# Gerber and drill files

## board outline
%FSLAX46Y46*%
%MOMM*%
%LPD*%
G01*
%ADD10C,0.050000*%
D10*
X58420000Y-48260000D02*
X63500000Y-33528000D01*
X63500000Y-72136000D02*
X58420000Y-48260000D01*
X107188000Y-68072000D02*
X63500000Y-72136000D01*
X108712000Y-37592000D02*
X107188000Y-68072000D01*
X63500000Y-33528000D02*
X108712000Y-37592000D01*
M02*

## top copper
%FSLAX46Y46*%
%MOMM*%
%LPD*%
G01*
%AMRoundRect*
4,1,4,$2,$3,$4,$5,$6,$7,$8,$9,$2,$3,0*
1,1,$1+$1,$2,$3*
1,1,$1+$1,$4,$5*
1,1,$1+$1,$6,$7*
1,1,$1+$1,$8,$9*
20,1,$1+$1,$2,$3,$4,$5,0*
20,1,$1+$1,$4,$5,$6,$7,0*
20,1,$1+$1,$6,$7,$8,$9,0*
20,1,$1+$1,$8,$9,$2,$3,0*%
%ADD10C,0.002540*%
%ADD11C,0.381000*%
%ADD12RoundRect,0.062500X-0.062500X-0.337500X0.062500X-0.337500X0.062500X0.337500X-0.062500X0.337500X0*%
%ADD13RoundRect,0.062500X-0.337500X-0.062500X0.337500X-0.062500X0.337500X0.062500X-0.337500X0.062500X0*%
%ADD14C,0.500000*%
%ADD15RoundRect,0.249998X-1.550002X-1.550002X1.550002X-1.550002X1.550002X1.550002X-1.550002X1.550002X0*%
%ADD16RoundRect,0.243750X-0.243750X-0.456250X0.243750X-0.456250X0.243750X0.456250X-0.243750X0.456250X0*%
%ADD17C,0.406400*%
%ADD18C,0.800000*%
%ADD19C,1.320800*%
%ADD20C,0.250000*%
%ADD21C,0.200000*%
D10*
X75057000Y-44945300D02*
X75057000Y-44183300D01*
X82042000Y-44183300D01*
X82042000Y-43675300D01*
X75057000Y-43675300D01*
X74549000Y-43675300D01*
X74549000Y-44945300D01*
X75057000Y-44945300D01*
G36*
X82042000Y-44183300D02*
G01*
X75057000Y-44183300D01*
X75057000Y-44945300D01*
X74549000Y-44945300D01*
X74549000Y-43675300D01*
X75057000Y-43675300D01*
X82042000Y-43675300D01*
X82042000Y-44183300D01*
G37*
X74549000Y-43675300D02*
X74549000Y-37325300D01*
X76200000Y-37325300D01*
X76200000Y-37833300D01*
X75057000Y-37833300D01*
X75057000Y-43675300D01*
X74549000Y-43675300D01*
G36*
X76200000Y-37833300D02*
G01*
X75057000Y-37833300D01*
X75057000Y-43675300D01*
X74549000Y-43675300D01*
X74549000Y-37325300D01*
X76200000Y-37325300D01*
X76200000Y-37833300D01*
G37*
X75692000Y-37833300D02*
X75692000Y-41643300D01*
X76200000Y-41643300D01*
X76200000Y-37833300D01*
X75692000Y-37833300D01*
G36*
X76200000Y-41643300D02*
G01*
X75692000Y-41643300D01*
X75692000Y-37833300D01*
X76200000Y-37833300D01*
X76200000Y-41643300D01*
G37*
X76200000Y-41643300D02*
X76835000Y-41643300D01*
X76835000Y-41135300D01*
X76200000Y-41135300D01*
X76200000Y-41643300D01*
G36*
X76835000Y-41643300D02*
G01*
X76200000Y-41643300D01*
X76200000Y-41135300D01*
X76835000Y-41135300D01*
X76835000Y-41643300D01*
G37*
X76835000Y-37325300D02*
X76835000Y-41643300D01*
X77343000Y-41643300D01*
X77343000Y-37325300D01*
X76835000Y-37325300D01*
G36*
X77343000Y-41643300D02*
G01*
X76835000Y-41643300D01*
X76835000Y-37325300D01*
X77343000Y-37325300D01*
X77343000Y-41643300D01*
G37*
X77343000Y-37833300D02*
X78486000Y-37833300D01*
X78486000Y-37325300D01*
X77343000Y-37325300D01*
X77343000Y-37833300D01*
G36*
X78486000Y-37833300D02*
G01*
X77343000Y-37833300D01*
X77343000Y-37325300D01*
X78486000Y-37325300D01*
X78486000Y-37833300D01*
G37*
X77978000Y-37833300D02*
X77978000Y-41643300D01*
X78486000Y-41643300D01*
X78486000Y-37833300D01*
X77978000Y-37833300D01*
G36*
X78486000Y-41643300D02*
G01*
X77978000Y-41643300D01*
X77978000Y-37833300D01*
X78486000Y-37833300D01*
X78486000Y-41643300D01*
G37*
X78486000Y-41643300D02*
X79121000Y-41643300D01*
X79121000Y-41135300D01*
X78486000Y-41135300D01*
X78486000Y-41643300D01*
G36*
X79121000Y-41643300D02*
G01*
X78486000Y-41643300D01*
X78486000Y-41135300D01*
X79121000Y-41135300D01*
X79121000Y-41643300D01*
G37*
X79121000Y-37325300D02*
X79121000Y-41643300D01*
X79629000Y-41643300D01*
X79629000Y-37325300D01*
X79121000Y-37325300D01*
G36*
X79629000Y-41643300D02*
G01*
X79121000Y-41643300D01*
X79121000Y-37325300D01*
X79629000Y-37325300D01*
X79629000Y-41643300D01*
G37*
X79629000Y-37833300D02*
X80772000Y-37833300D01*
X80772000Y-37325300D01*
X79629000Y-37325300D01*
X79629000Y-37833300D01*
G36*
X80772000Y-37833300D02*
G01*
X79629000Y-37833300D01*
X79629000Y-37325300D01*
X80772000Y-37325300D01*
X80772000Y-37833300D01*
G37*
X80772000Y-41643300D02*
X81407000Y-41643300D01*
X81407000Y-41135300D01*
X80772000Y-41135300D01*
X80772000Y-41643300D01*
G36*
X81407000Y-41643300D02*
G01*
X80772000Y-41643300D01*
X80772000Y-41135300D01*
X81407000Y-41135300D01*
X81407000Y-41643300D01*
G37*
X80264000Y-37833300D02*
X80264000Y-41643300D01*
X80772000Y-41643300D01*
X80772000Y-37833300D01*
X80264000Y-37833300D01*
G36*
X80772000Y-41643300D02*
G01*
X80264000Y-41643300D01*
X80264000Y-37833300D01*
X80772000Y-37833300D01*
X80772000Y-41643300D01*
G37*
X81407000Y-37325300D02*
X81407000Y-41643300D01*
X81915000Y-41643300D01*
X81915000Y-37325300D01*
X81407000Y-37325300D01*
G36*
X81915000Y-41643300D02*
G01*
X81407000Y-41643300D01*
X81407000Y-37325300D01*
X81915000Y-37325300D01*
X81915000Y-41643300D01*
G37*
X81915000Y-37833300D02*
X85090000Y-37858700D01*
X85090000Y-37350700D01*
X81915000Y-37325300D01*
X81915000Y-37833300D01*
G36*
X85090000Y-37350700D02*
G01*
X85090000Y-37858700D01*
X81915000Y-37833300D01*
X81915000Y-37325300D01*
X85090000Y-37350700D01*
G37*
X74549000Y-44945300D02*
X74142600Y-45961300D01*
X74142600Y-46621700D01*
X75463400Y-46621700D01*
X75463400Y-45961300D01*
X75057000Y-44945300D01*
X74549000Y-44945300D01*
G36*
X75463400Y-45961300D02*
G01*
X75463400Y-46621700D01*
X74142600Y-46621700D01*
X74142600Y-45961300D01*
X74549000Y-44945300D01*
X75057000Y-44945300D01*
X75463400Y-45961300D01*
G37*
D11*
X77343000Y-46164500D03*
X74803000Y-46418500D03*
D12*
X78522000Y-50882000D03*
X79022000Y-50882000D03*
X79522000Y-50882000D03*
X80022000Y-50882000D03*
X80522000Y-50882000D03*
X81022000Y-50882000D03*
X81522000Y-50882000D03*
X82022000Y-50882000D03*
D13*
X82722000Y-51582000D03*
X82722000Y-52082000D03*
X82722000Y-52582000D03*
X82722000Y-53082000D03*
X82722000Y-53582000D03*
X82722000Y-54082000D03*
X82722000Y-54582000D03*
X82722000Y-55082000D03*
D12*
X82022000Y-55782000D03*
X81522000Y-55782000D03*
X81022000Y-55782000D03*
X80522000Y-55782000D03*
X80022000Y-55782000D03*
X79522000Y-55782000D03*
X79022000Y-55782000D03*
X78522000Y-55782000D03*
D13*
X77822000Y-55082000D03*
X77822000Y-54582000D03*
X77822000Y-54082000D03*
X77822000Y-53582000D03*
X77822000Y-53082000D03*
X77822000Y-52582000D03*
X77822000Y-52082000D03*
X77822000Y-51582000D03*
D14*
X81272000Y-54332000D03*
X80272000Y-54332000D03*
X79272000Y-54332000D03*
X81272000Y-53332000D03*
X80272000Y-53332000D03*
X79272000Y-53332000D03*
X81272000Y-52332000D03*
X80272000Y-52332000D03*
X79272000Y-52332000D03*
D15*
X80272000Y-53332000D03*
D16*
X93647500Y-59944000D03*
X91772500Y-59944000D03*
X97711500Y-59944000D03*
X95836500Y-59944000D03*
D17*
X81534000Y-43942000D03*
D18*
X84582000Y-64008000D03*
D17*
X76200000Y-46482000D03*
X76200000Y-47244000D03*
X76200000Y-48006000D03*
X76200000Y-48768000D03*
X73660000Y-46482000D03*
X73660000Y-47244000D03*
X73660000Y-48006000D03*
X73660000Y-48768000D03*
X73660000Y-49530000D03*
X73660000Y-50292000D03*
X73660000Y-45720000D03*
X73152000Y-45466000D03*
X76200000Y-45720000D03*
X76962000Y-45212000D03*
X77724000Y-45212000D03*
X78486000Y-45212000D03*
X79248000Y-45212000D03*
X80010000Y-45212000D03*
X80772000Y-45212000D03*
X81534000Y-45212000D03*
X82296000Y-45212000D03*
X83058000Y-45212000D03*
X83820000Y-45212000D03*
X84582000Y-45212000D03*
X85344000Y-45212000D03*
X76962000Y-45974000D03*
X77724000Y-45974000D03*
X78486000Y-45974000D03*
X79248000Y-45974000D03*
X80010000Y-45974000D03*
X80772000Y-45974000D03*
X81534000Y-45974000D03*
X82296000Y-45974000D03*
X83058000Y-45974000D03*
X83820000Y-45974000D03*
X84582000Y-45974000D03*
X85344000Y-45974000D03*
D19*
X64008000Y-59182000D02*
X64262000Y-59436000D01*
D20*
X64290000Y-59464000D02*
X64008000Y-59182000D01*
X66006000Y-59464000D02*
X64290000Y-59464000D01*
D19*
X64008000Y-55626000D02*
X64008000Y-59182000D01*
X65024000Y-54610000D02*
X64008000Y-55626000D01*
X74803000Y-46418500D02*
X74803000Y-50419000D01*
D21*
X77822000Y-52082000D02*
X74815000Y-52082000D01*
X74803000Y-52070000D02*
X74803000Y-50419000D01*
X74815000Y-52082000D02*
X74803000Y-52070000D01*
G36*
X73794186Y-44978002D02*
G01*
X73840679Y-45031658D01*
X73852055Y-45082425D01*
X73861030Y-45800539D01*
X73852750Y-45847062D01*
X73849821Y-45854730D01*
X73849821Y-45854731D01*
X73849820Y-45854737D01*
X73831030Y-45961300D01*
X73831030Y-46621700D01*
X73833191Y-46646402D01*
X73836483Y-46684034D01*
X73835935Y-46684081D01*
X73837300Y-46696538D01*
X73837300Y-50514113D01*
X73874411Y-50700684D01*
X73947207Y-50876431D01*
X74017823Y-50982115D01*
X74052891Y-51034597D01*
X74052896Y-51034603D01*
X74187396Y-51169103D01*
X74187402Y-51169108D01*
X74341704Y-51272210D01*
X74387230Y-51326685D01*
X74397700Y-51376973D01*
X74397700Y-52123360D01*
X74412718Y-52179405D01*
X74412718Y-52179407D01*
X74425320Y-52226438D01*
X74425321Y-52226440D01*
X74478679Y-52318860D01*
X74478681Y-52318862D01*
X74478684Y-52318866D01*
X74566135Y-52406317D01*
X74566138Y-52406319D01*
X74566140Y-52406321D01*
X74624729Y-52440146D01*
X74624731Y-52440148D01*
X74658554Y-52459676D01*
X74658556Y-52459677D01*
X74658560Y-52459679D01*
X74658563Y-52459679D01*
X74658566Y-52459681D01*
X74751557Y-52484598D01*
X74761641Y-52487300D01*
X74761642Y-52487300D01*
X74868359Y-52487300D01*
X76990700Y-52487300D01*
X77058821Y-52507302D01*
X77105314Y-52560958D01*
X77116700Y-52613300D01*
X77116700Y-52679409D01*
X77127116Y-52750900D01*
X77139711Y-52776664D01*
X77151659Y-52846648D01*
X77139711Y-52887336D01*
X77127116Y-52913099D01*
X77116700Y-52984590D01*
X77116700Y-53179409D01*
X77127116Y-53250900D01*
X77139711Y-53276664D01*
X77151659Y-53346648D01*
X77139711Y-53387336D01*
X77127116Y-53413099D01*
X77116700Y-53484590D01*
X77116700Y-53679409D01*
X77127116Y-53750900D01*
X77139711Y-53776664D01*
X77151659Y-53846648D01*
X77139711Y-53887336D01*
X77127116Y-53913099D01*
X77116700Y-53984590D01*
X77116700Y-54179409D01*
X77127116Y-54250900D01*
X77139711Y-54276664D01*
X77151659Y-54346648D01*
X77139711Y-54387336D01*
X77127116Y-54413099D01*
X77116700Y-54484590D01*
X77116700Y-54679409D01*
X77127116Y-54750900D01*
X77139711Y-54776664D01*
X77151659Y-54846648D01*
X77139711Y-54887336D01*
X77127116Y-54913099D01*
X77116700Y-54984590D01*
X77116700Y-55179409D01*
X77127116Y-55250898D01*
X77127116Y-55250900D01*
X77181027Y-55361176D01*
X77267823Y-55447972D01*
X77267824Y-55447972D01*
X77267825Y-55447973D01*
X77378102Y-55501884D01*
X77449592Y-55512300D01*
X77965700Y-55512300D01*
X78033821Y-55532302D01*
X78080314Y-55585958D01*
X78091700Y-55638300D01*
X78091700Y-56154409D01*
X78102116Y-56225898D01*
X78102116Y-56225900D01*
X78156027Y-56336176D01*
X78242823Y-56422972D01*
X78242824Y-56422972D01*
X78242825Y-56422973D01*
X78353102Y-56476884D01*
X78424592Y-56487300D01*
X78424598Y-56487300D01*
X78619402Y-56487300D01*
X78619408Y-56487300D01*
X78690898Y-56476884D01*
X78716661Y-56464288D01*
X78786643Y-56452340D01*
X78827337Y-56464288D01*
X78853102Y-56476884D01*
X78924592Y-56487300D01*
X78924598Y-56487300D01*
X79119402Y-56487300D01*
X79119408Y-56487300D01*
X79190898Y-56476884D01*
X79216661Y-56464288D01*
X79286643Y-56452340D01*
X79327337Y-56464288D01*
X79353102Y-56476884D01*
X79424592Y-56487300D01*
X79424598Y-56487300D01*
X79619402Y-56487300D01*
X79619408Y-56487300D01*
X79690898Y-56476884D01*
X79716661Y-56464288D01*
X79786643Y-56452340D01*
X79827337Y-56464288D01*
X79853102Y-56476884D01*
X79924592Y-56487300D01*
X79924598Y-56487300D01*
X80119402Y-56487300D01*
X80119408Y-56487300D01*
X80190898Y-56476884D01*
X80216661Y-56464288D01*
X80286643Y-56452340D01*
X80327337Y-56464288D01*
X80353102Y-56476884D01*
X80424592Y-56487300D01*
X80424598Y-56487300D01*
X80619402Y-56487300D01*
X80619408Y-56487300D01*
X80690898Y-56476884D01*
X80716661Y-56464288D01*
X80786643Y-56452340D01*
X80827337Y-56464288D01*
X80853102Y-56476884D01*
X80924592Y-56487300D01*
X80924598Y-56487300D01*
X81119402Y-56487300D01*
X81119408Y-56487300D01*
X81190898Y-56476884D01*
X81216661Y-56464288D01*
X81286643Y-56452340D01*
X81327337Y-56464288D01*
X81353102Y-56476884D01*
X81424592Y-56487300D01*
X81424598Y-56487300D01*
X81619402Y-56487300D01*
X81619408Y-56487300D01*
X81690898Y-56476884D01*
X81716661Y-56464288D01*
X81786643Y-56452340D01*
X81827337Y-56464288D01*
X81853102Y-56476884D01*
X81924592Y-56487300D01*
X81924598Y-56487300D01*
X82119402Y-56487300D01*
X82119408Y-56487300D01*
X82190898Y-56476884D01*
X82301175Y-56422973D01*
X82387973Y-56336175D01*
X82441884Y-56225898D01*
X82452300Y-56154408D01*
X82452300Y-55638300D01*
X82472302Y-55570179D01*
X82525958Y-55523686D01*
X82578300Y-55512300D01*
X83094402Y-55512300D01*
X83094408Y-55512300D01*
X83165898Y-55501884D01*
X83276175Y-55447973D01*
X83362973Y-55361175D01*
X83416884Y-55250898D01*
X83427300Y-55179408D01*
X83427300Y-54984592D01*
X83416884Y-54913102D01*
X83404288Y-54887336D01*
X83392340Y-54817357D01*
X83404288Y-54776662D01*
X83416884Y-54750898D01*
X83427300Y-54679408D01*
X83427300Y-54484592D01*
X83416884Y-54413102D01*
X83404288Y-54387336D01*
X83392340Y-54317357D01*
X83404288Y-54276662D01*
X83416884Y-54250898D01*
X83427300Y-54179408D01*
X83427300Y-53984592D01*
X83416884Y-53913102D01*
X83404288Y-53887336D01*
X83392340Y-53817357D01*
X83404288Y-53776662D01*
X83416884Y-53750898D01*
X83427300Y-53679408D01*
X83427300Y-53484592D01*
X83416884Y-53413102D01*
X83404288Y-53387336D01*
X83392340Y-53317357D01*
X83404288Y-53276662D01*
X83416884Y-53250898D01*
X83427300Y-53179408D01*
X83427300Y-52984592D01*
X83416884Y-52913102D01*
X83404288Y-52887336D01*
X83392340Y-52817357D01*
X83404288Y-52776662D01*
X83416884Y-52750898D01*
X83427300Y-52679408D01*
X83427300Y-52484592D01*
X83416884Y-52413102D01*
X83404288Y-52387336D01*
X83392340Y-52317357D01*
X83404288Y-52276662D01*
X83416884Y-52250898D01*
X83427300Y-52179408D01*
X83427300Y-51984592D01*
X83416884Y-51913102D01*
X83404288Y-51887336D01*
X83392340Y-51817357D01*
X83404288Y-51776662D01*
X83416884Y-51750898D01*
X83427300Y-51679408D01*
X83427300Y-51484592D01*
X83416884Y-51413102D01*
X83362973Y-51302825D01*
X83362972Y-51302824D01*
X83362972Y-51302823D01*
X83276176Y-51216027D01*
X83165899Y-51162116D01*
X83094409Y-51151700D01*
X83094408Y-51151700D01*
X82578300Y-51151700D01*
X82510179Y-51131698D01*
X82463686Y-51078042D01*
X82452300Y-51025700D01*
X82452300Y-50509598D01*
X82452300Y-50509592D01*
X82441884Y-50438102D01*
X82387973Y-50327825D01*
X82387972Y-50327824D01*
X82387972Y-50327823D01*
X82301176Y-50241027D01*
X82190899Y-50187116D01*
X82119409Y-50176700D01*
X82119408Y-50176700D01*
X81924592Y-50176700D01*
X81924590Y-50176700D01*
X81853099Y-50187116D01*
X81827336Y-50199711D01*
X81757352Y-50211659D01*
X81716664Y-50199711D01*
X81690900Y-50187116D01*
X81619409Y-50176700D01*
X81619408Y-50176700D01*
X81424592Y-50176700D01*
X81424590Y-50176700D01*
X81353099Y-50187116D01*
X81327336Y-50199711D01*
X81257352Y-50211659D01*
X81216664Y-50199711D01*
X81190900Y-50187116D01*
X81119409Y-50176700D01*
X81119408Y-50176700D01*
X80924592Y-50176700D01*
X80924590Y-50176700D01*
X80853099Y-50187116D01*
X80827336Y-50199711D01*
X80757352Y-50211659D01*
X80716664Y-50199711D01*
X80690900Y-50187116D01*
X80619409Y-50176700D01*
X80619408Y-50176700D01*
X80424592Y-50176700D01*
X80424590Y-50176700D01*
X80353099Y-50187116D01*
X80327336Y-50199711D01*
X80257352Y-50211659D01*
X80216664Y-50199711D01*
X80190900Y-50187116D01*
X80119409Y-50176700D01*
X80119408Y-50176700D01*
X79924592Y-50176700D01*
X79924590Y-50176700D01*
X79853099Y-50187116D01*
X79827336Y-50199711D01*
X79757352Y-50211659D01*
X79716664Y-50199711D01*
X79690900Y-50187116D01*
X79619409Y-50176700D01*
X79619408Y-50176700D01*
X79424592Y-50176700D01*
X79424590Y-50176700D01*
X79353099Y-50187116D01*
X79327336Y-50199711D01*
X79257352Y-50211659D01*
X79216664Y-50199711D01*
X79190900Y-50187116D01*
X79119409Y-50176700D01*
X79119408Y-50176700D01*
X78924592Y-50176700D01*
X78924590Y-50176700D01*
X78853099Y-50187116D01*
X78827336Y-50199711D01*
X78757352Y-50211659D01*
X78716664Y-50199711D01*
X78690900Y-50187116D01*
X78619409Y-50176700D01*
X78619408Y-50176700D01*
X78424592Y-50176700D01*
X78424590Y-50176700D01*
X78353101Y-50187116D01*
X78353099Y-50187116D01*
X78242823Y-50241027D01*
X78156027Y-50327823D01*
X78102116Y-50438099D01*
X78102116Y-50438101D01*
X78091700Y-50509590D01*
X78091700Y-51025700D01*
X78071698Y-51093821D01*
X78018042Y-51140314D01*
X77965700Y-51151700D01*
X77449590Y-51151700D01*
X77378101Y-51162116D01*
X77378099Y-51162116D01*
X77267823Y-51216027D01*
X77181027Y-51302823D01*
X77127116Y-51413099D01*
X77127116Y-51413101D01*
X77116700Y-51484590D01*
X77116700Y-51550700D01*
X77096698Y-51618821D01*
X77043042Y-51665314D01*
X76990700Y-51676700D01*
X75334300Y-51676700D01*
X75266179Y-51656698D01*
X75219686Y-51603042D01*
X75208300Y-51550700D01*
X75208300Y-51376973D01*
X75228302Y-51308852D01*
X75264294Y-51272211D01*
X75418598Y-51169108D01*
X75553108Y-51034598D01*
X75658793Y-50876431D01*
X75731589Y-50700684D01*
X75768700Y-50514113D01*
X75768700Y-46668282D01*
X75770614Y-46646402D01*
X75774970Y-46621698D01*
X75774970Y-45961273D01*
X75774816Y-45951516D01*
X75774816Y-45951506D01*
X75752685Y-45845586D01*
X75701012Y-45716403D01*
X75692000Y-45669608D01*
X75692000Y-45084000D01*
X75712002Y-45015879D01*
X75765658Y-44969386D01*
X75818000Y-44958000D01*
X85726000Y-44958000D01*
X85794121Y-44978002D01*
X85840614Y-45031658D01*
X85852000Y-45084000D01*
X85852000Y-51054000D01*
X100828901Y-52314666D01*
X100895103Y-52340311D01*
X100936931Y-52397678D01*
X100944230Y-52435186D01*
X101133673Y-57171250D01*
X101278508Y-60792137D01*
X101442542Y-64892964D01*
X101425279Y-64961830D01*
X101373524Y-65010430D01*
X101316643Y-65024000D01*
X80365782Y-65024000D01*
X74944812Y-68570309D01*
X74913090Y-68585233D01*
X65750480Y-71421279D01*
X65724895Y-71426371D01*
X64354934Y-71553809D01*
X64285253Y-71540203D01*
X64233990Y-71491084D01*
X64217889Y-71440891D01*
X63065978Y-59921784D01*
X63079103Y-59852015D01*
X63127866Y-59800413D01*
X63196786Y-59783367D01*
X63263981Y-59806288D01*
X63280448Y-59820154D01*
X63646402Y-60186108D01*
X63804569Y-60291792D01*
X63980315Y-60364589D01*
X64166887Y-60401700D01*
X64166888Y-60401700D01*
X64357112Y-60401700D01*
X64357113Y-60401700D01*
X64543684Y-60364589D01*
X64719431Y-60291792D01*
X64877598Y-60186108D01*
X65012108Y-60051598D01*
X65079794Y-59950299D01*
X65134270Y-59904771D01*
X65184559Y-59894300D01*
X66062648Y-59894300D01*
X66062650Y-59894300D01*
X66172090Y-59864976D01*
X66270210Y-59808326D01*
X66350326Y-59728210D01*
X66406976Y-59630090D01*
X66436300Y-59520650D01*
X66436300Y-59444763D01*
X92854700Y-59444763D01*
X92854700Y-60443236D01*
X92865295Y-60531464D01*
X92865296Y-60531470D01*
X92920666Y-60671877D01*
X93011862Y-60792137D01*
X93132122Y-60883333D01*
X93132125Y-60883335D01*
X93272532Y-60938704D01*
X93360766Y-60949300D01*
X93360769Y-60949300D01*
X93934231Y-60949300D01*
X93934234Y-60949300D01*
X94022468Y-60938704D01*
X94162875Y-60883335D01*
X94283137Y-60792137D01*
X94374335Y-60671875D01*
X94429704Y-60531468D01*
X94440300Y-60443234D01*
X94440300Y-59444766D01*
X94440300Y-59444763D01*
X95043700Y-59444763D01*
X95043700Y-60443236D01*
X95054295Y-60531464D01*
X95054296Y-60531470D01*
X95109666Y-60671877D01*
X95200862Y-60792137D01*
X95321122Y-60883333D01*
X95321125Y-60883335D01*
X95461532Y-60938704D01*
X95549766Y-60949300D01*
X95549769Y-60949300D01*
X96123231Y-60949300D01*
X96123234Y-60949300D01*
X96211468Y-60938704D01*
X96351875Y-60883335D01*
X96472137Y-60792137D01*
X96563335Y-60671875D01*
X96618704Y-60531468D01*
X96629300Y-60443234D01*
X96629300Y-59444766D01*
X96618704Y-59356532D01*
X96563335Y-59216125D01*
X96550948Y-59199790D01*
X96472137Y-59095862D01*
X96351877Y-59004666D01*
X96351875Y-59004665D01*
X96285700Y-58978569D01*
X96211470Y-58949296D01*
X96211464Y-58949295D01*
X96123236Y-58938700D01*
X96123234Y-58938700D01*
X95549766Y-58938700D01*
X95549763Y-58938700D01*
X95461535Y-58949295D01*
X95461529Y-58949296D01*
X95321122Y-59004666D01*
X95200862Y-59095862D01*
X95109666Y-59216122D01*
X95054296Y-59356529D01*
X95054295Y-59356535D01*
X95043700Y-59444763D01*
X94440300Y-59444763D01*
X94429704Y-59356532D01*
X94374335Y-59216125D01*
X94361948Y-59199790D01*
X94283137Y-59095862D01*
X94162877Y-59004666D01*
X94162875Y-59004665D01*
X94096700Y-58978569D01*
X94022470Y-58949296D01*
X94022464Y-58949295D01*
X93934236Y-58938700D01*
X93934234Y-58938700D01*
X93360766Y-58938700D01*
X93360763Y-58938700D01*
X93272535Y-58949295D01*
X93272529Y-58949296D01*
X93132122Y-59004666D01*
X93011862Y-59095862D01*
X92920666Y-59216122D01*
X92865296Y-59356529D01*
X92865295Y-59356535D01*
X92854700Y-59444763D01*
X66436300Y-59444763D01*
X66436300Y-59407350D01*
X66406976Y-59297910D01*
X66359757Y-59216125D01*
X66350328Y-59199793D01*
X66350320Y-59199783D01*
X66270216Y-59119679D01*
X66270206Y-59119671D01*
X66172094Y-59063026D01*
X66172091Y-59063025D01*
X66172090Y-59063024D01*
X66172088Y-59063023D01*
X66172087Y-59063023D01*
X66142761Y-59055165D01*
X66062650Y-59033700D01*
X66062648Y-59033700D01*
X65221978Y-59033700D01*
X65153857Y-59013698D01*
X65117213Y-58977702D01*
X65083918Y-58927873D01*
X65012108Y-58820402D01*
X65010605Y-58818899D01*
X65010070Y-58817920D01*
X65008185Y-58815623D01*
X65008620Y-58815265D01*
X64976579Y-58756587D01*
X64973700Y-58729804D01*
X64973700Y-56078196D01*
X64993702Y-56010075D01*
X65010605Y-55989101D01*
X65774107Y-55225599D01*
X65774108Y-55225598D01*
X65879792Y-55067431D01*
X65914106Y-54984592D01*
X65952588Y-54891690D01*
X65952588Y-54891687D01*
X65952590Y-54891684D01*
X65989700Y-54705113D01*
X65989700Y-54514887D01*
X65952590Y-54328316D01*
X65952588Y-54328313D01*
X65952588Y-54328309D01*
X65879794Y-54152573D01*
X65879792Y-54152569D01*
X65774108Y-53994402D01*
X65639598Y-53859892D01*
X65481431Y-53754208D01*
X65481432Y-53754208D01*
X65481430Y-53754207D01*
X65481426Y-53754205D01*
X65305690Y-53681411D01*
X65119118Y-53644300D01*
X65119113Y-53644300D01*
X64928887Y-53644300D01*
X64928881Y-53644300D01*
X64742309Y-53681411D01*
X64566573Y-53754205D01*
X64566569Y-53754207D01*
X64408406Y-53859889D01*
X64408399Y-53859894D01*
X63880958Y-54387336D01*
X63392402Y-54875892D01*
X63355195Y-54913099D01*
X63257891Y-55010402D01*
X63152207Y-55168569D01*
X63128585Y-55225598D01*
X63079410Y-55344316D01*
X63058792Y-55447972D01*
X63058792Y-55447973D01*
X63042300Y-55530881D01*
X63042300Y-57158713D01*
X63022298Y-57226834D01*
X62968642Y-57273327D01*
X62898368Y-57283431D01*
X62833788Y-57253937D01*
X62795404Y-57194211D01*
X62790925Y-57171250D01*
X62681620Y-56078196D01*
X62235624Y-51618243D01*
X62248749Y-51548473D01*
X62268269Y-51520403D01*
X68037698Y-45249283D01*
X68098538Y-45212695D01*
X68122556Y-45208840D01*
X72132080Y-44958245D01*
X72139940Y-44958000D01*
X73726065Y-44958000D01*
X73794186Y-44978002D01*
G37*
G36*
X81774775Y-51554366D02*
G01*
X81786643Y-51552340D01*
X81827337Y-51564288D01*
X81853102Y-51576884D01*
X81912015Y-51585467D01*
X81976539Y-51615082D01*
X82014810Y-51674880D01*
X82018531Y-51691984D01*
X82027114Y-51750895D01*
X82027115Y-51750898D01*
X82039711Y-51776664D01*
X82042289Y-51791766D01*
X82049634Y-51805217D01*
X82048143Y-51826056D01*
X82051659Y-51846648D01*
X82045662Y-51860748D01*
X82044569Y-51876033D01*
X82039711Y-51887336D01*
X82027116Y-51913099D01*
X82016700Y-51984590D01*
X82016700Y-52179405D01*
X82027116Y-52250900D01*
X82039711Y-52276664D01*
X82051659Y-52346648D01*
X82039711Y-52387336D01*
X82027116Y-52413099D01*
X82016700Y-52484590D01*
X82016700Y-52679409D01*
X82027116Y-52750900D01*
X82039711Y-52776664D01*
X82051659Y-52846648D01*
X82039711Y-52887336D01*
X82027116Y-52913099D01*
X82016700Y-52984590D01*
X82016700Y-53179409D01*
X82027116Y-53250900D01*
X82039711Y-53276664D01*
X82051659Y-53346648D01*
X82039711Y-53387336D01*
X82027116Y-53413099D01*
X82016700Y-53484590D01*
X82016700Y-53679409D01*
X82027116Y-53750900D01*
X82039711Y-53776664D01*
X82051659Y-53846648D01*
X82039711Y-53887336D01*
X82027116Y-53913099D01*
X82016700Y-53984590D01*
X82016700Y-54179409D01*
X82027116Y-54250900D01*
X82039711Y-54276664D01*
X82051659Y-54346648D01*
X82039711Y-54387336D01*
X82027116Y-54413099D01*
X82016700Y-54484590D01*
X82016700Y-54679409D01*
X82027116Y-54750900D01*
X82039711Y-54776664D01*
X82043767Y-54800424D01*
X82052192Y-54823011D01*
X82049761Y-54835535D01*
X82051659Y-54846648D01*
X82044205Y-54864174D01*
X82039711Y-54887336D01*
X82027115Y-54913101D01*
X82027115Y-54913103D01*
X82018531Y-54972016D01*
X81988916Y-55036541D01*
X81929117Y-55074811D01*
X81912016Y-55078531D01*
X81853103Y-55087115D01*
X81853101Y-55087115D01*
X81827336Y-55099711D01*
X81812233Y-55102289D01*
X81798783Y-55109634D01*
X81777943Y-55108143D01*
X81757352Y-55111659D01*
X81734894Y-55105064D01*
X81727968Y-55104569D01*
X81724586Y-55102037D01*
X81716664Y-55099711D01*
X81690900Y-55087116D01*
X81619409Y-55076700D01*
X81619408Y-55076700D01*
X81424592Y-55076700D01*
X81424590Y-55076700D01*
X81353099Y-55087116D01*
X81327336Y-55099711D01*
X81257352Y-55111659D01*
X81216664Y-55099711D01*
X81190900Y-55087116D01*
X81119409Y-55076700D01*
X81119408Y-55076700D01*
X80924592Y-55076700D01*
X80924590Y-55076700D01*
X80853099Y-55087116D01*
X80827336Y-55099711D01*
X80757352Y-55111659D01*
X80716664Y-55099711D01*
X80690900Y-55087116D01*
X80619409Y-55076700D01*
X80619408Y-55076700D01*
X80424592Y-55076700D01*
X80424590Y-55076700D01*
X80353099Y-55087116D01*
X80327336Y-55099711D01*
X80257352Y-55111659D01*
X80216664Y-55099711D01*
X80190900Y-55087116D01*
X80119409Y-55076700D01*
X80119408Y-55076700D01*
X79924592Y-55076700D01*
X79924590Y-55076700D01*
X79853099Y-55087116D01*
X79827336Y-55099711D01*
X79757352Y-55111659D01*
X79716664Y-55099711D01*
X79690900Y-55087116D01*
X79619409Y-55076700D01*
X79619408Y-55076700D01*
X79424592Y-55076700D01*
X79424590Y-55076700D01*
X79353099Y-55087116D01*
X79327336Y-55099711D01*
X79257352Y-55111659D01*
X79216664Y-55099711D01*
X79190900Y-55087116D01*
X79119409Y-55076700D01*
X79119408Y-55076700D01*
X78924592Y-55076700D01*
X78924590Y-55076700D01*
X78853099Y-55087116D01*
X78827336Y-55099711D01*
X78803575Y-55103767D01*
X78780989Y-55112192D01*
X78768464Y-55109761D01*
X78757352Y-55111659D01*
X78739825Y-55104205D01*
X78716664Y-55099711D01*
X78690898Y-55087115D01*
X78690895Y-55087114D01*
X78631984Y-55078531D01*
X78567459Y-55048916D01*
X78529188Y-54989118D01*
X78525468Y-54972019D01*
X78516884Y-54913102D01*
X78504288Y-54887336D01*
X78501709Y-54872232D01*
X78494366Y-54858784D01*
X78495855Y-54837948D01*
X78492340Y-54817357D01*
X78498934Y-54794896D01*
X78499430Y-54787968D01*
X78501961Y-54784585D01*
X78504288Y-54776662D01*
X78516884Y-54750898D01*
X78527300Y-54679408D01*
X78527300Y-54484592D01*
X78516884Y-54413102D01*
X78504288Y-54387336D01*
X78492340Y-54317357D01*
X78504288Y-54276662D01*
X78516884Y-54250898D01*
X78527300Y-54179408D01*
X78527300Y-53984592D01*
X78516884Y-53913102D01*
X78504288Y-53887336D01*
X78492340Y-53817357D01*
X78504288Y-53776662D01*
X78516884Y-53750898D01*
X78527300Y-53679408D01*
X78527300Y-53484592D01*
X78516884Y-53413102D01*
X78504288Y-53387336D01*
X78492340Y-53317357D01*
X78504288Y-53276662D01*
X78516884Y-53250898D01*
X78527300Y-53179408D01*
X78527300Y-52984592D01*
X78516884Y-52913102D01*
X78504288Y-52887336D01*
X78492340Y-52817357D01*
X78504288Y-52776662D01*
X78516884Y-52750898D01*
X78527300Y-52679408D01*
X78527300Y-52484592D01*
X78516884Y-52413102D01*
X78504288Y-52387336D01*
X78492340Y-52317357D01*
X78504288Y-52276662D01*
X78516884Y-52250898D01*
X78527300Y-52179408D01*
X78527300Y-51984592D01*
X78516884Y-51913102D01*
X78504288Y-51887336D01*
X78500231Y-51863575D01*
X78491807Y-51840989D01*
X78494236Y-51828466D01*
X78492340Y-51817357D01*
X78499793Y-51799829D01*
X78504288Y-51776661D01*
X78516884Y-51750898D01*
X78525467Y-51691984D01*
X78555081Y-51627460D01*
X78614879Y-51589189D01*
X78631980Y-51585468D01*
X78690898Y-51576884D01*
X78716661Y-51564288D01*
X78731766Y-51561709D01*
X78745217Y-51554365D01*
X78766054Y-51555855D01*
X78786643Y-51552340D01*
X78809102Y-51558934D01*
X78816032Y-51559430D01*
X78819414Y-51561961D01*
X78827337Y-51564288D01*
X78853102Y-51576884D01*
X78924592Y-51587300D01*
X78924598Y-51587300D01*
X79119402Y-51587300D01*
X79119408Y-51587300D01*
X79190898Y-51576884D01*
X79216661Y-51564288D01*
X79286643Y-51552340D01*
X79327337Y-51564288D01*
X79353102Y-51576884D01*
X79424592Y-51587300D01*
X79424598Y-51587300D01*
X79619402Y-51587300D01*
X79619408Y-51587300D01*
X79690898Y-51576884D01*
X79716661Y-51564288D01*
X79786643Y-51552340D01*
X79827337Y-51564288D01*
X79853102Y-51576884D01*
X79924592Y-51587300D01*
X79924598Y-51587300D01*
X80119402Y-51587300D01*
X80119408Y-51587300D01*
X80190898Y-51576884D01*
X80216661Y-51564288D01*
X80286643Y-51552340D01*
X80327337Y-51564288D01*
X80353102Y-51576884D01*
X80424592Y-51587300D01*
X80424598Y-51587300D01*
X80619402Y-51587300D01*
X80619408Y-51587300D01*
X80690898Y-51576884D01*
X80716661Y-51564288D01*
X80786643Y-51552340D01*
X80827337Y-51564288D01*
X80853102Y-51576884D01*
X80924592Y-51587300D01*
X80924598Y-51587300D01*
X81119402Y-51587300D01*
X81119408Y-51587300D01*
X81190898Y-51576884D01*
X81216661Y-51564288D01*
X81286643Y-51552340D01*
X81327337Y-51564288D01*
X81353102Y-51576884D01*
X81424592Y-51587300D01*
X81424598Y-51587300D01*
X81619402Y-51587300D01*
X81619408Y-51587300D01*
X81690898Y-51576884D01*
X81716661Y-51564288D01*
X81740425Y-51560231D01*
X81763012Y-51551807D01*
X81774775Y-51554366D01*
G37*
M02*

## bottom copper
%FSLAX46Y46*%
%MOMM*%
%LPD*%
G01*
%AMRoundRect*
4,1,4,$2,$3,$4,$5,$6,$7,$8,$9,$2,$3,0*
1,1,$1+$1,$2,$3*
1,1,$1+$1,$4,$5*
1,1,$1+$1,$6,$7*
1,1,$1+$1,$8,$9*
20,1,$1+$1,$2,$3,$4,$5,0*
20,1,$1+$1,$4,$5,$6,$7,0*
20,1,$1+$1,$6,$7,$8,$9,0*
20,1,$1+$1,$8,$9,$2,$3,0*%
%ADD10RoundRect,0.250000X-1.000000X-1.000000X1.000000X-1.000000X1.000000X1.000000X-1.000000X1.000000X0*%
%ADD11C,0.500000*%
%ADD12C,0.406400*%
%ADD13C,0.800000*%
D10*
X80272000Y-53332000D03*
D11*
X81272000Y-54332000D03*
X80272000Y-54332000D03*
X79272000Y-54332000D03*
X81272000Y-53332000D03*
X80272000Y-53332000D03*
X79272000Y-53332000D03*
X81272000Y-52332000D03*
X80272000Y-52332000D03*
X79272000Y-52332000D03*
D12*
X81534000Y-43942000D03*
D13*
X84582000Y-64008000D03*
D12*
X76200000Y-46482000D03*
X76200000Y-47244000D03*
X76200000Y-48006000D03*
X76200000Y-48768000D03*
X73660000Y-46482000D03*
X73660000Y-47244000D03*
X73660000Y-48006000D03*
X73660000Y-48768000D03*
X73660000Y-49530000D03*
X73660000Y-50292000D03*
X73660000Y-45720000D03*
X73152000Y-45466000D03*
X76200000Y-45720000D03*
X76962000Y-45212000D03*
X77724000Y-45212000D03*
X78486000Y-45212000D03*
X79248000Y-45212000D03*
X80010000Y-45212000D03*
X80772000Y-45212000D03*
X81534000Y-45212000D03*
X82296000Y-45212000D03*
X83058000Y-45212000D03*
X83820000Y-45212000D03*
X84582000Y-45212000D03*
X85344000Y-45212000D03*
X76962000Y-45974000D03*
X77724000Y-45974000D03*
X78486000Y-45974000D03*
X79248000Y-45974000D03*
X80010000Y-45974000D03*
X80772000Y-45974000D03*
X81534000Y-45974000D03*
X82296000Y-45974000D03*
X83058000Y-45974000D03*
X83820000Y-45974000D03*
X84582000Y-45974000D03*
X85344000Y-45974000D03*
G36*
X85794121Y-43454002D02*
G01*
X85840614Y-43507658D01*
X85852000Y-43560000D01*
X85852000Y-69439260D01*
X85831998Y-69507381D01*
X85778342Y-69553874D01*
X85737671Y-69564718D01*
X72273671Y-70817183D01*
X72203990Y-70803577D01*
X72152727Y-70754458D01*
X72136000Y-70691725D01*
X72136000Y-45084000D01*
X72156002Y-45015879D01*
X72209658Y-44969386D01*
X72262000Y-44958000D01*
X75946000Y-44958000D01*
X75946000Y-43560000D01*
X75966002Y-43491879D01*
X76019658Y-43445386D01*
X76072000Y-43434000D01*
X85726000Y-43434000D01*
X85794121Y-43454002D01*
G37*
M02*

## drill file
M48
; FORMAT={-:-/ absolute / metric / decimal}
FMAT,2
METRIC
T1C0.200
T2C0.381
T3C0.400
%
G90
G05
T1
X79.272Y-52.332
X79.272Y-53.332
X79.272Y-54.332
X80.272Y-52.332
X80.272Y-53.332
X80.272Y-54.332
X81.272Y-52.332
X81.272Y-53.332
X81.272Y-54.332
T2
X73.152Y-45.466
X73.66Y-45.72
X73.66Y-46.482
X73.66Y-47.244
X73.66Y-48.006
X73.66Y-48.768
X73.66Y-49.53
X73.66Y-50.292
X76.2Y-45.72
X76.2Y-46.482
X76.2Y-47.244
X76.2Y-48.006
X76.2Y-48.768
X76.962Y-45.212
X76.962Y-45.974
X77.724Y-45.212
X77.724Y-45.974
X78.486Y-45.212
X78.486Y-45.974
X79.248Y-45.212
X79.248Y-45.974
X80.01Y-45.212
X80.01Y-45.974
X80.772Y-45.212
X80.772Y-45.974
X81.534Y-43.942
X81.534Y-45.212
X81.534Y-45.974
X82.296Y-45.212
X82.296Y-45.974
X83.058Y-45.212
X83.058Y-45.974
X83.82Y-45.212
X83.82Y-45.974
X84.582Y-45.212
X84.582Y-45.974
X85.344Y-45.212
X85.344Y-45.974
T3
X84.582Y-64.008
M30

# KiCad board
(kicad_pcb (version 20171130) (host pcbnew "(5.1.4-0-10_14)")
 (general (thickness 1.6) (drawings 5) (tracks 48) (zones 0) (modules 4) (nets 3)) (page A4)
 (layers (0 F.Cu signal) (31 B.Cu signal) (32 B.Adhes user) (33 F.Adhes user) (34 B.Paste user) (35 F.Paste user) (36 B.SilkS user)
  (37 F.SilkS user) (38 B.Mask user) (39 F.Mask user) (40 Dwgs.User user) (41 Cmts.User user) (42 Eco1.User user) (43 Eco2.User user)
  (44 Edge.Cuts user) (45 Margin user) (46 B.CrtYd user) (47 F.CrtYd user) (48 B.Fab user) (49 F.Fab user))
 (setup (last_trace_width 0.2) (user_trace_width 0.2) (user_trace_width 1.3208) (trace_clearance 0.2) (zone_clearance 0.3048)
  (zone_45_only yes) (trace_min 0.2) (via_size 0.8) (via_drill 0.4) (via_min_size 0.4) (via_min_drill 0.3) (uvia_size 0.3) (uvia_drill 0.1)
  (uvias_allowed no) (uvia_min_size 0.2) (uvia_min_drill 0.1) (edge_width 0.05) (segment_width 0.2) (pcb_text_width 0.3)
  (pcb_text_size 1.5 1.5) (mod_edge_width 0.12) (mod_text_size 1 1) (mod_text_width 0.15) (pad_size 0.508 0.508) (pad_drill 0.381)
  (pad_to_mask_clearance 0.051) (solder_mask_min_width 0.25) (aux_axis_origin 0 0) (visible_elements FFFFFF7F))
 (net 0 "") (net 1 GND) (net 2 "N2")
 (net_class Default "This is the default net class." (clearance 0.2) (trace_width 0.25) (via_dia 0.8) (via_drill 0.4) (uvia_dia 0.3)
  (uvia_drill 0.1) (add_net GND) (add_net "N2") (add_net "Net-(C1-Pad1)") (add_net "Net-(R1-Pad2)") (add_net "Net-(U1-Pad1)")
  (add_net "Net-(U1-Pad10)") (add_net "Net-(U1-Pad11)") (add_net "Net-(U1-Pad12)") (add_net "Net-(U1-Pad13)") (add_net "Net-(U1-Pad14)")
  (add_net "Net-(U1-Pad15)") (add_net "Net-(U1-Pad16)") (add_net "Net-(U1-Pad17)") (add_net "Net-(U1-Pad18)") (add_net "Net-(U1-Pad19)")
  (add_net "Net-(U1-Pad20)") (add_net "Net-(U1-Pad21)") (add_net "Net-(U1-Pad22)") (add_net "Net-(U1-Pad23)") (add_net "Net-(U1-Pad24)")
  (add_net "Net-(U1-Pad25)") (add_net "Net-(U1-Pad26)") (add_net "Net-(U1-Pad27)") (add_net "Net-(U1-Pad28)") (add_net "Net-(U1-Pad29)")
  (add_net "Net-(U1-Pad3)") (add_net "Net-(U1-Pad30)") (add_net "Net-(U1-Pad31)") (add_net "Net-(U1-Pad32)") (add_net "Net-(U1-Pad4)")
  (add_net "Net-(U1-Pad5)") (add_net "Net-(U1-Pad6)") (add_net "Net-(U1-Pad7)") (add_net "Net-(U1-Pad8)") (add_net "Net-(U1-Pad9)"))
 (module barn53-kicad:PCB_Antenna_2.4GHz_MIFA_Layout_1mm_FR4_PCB (layer F.Cu) (at 74.803 46.4185)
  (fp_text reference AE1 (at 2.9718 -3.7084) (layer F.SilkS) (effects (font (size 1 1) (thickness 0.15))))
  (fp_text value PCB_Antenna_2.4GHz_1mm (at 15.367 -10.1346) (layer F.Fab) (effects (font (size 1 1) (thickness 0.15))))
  (fp_poly
   (pts (xy 0.254 -1.4732) (xy 0.254 -2.2352) (xy 7.239 -2.2352) (xy 7.239 -2.7432) (xy 0.254 -2.7432) (xy -0.254 -2.7432)
    (xy -0.254 -1.4732))
   (layer F.Cu) (width 0.00254))
  (fp_poly
   (pts (xy -0.254 -2.7432) (xy -0.254 -9.0932) (xy 1.397 -9.0932) (xy 1.397 -8.5852) (xy 0.254 -8.5852) (xy 0.254 -2.7432)) (layer F.Cu)
   (width 0.00254))
  (fp_poly (pts (xy 0.889 -8.5852) (xy 0.889 -4.7752) (xy 1.397 -4.7752) (xy 1.397 -8.5852)) (layer F.Cu) (width 0.00254))
  (fp_poly (pts (xy 1.397 -4.7752) (xy 2.032 -4.7752) (xy 2.032 -5.2832) (xy 1.397 -5.2832)) (layer F.Cu) (width 0.00254))
  (fp_poly (pts (xy 2.032 -9.0932) (xy 2.032 -4.7752) (xy 2.54 -4.7752) (xy 2.54 -9.0932)) (layer F.Cu) (width 0.00254))
  (fp_poly (pts (xy 2.54 -8.5852) (xy 3.683 -8.5852) (xy 3.683 -9.0932) (xy 2.54 -9.0932)) (layer F.Cu) (width 0.00254))
  (fp_poly (pts (xy 3.175 -8.5852) (xy 3.175 -4.7752) (xy 3.683 -4.7752) (xy 3.683 -8.5852)) (layer F.Cu) (width 0.00254))
  (fp_poly (pts (xy 3.683 -4.7752) (xy 4.318 -4.7752) (xy 4.318 -5.2832) (xy 3.683 -5.2832)) (layer F.Cu) (width 0.00254))
  (fp_poly (pts (xy 4.318 -9.0932) (xy 4.318 -4.7752) (xy 4.826 -4.7752) (xy 4.826 -9.0932)) (layer F.Cu) (width 0.00254))
  (fp_poly (pts (xy 4.826 -8.5852) (xy 5.969 -8.5852) (xy 5.969 -9.0932) (xy 4.826 -9.0932)) (layer F.Cu) (width 0.00254))
  (fp_poly (pts (xy 5.969 -4.7752) (xy 6.604 -4.7752) (xy 6.604 -5.2832) (xy 5.969 -5.2832)) (layer F.Cu) (width 0.00254))
  (fp_poly (pts (xy 5.461 -8.5852) (xy 5.461 -4.7752) (xy 5.969 -4.7752) (xy 5.969 -8.5852)) (layer F.Cu) (width 0.00254))
  (fp_poly (pts (xy 6.604 -9.0932) (xy 6.604 -4.7752) (xy 7.112 -4.7752) (xy 7.112 -9.0932)) (layer F.Cu) (width 0.00254))
  (fp_poly (pts (xy 7.112 -8.5852) (xy 10.287 -8.5598) (xy 10.287 -9.0678) (xy 7.112 -9.0932)) (layer F.Cu) (width 0.00254))
  (fp_poly
   (pts (xy -0.254 -1.4732) (xy -0.6604 -0.4572) (xy -0.6604 0.2032) (xy 0.6604 0.2032) (xy 0.6604 -0.4572) (xy 0.254 -1.4732)) (layer F.Cu)
   (width 0.00254))
  (pad 2 connect circle (at 2.54 -0.254) (size 0.381 0.381) (layers F.Cu) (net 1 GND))
  (pad 1 connect circle (at 0 0) (size 0.381 0.381) (layers F.Cu) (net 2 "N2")))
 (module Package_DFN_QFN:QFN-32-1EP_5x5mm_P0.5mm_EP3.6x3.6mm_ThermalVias (layer F.Cu) (at 80.272 53.332)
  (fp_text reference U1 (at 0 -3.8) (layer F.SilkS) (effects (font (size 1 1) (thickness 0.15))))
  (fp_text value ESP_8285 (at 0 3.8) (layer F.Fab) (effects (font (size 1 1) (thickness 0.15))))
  (pad 32 smd roundrect (at -1.75 -2.45) (size 0.25 0.8) (layers F.Cu F.Paste F.Mask) (roundrect_rratio 0.25))
  (pad 31 smd roundrect (at -1.25 -2.45) (size 0.25 0.8) (layers F.Cu F.Paste F.Mask) (roundrect_rratio 0.25))
  (pad 30 smd roundrect (at -0.75 -2.45) (size 0.25 0.8) (layers F.Cu F.Paste F.Mask) (roundrect_rratio 0.25))
  (pad 29 smd roundrect (at -0.25 -2.45) (size 0.25 0.8) (layers F.Cu F.Paste F.Mask) (roundrect_rratio 0.25))
  (pad 28 smd roundrect (at 0.25 -2.45) (size 0.25 0.8) (layers F.Cu F.Paste F.Mask) (roundrect_rratio 0.25))
  (pad 27 smd roundrect (at 0.75 -2.45) (size 0.25 0.8) (layers F.Cu F.Paste F.Mask) (roundrect_rratio 0.25))
  (pad 26 smd roundrect (at 1.25 -2.45) (size 0.25 0.8) (layers F.Cu F.Paste F.Mask) (roundrect_rratio 0.25))
  (pad 25 smd roundrect (at 1.75 -2.45) (size 0.25 0.8) (layers F.Cu F.Paste F.Mask) (roundrect_rratio 0.25))
  (pad 24 smd roundrect (at 2.45 -1.75) (size 0.8 0.25) (layers F.Cu F.Paste F.Mask) (roundrect_rratio 0.25))
  (pad 23 smd roundrect (at 2.45 -1.25) (size 0.8 0.25) (layers F.Cu F.Paste F.Mask) (roundrect_rratio 0.25))
  (pad 22 smd roundrect (at 2.45 -0.75) (size 0.8 0.25) (layers F.Cu F.Paste F.Mask) (roundrect_rratio 0.25))
  (pad 21 smd roundrect (at 2.45 -0.25) (size 0.8 0.25) (layers F.Cu F.Paste F.Mask) (roundrect_rratio 0.25))
  (pad 20 smd roundrect (at 2.45 0.25) (size 0.8 0.25) (layers F.Cu F.Paste F.Mask) (roundrect_rratio 0.25))
  (pad 19 smd roundrect (at 2.45 0.75) (size 0.8 0.25) (layers F.Cu F.Paste F.Mask) (roundrect_rratio 0.25))
  (pad 18 smd roundrect (at 2.45 1.25) (size 0.8 0.25) (layers F.Cu F.Paste F.Mask) (roundrect_rratio 0.25))
  (pad 17 smd roundrect (at 2.45 1.75) (size 0.8 0.25) (layers F.Cu F.Paste F.Mask) (roundrect_rratio 0.25))
  (pad 16 smd roundrect (at 1.75 2.45) (size 0.25 0.8) (layers F.Cu F.Paste F.Mask) (roundrect_rratio 0.25))
  (pad 15 smd roundrect (at 1.25 2.45) (size 0.25 0.8) (layers F.Cu F.Paste F.Mask) (roundrect_rratio 0.25))
  (pad 14 smd roundrect (at 0.75 2.45) (size 0.25 0.8) (layers F.Cu F.Paste F.Mask) (roundrect_rratio 0.25))
  (pad 13 smd roundrect (at 0.25 2.45) (size 0.25 0.8) (layers F.Cu F.Paste F.Mask) (roundrect_rratio 0.25))
  (pad 12 smd roundrect (at -0.25 2.45) (size 0.25 0.8) (layers F.Cu F.Paste F.Mask) (roundrect_rratio 0.25))
  (pad 11 smd roundrect (at -0.75 2.45) (size 0.25 0.8) (layers F.Cu F.Paste F.Mask) (roundrect_rratio 0.25))
  (pad 10 smd roundrect (at -1.25 2.45) (size 0.25 0.8) (layers F.Cu F.Paste F.Mask) (roundrect_rratio 0.25))
  (pad 9 smd roundrect (at -1.75 2.45) (size 0.25 0.8) (layers F.Cu F.Paste F.Mask) (roundrect_rratio 0.25))
  (pad 8 smd roundrect (at -2.45 1.75) (size 0.8 0.25) (layers F.Cu F.Paste F.Mask) (roundrect_rratio 0.25))
  (pad 7 smd roundrect (at -2.45 1.25) (size 0.8 0.25) (layers F.Cu F.Paste F.Mask) (roundrect_rratio 0.25))
  (pad 6 smd roundrect (at -2.45 0.75) (size 0.8 0.25) (layers F.Cu F.Paste F.Mask) (roundrect_rratio 0.25))
  (pad 5 smd roundrect (at -2.45 0.25) (size 0.8 0.25) (layers F.Cu F.Paste F.Mask) (roundrect_rratio 0.25))
  (pad 4 smd roundrect (at -2.45 -0.25) (size 0.8 0.25) (layers F.Cu F.Paste F.Mask) (roundrect_rratio 0.25))
  (pad 3 smd roundrect (at -2.45 -0.75) (size 0.8 0.25) (layers F.Cu F.Paste F.Mask) (roundrect_rratio 0.25))
  (pad 2 smd roundrect (at -2.45 -1.25) (size 0.8 0.25) (layers F.Cu F.Paste F.Mask) (roundrect_rratio 0.25) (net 2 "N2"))
  (pad 1 smd roundrect (at -2.45 -1.75) (size 0.8 0.25) (layers F.Cu F.Paste F.Mask) (roundrect_rratio 0.25))
  (pad "" smd custom (at 1.4 1.4) (size 0.554596 0.554596) (layers F.Paste) (options (clearance outline) (anchor circle)) (primitives))
  (pad "" smd custom (at 1.4 -1.4) (size 0.554596 0.554596) (layers F.Paste) (options (clearance outline) (anchor circle)) (primitives))
  (pad "" smd custom (at -1.4 1.4) (size 0.554596 0.554596) (layers F.Paste) (options (clearance outline) (anchor circle)) (primitives))
  (pad "" smd custom (at -1.4 -1.4) (size 0.554596 0.554596) (layers F.Paste) (options (clearance outline) (anchor circle)) (primitives))
  (pad "" smd custom (at 0.5 1.4) (size 0.568298 0.568298) (layers F.Paste) (options (clearance outline) (anchor circle)) (primitives))
  (pad "" smd custom (at -0.5 1.4) (size 0.568298 0.568298) (layers F.Paste) (options (clearance outline) (anchor circle)) (primitives))
  (pad "" smd custom (at 0.5 -1.4) (size 0.568298 0.568298) (layers F.Paste) (options (clearance outline) (anchor circle)) (primitives))
  (pad "" smd custom (at -0.5 -1.4) (size 0.568298 0.568298) (layers F.Paste) (options (clearance outline) (anchor circle)) (primitives))
  (pad "" smd custom (at 1.4 0.5) (size 0.568298 0.568298) (layers F.Paste) (options (clearance outline) (anchor circle)) (primitives))
  (pad "" smd custom (at 1.4 -0.5) (size 0.568298 0.568298) (layers F.Paste) (options (clearance outline) (anchor circle)) (primitives))
  (pad "" smd custom (at -1.4 0.5) (size 0.568298 0.568298) (layers F.Paste) (options (clearance outline) (anchor circle)) (primitives))
  (pad "" smd custom (at -1.4 -0.5) (size 0.568298 0.568298) (layers F.Paste) (options (clearance outline) (anchor circle)) (primitives))
  (pad "" smd roundrect (at 0.5 0.5) (size 0.806226 0.806226) (layers F.Paste) (roundrect_rratio 0.25))
  (pad "" smd roundrect (at 0.5 -0.5) (size 0.806226 0.806226) (layers F.Paste) (roundrect_rratio 0.25))
  (pad "" smd roundrect (at -0.5 0.5) (size 0.806226 0.806226) (layers F.Paste) (roundrect_rratio 0.25))
  (pad "" smd roundrect (at -0.5 -0.5) (size 0.806226 0.806226) (layers F.Paste) (roundrect_rratio 0.25))
  (pad 33 smd roundrect (at 0 0) (size 2.5 2.5) (layers B.Cu) (roundrect_rratio 0.1) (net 1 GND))
  (pad 33 thru_hole circle (at 1 1) (size 0.5 0.5) (drill 0.2) (layers *.Cu) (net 1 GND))
  (pad 33 thru_hole circle (at 0 1) (size 0.5 0.5) (drill 0.2) (layers *.Cu) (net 1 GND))
  (pad 33 thru_hole circle (at -1 1) (size 0.5 0.5) (drill 0.2) (layers *.Cu) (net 1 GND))
  (pad 33 thru_hole circle (at 1 0) (size 0.5 0.5) (drill 0.2) (layers *.Cu) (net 1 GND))
  (pad 33 thru_hole circle (at 0 0) (size 0.5 0.5) (drill 0.2) (layers *.Cu) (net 1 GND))
  (pad 33 thru_hole circle (at -1 0) (size 0.5 0.5) (drill 0.2) (layers *.Cu) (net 1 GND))
  (pad 33 thru_hole circle (at 1 -1) (size 0.5 0.5) (drill 0.2) (layers *.Cu) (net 1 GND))
  (pad 33 thru_hole circle (at 0 -1) (size 0.5 0.5) (drill 0.2) (layers *.Cu) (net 1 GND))
  (pad 33 thru_hole circle (at -1 -1) (size 0.5 0.5) (drill 0.2) (layers *.Cu) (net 1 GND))
  (pad 33 smd roundrect (at 0 0) (size 3.6 3.6) (layers F.Cu F.Mask) (roundrect_rratio 0.06944400000000001) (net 1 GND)))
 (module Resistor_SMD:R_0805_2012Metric (layer F.Cu) (at 92.71 59.944)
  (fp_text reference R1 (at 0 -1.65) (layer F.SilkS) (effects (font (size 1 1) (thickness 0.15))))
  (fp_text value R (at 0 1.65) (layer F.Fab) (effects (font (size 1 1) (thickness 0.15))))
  (pad 2 smd roundrect (at 0.9375 0) (size 0.975 1.4) (layers F.Cu F.Paste F.Mask) (roundrect_rratio 0.25))
  (pad 1 smd roundrect (at -0.9375 0) (size 0.975 1.4) (layers F.Cu F.Paste F.Mask) (roundrect_rratio 0.25) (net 1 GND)))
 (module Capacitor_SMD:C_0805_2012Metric (layer F.Cu) (at 96.774 59.944)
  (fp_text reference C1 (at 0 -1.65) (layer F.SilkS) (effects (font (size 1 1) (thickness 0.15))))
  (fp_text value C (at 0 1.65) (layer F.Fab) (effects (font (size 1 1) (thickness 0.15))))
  (pad 2 smd roundrect (at 0.9375 0) (size 0.975 1.4) (layers F.Cu F.Paste F.Mask) (roundrect_rratio 0.25) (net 1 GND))
  (pad 1 smd roundrect (at -0.9375 0) (size 0.975 1.4) (layers F.Cu F.Paste F.Mask) (roundrect_rratio 0.25)))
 (gr_line (start 58.42 48.26) (end 63.5 33.528) (layer Edge.Cuts) (width 0.05))
 (gr_line (start 63.5 72.136) (end 58.42 48.26) (layer Edge.Cuts) (width 0.05))
 (gr_line (start 107.188 68.072) (end 63.5 72.136) (layer Edge.Cuts) (width 0.05))
 (gr_line (start 108.712 37.592) (end 107.188 68.072) (layer Edge.Cuts) (width 0.05))
 (gr_line (start 63.5 33.528) (end 108.712 37.592) (layer Edge.Cuts) (width 0.05))
 (segment (start 64.008 59.182) (end 64.262 59.436) (width 1.3208) (layer F.Cu) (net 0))
 (segment (start 64.29 59.464) (end 64.008 59.182) (width 0.25) (layer F.Cu) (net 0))
 (segment (start 66.006 59.464) (end 64.29 59.464) (width 0.25) (layer F.Cu) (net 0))
 (segment (start 64.008 55.626) (end 64.008 59.182) (width 1.3208) (layer F.Cu) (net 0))
 (segment (start 65.024 54.61) (end 64.008 55.626) (width 1.3208) (layer F.Cu) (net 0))
 (segment (start 74.803 46.4185) (end 74.803 50.419) (width 1.3208) (layer F.Cu) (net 2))
 (segment (start 77.822 52.082) (end 74.815 52.082) (width 0.2) (layer F.Cu) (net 2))
 (segment (start 74.803 52.07) (end 74.803 50.419) (width 0.2) (layer F.Cu) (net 2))
 (segment (start 74.815 52.082) (end 74.803 52.07) (width 0.2) (layer F.Cu) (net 2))
 (via (at 81.534 43.942) (size 0.4064) (drill 0.381) (layers F.Cu B.Cu) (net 1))
 (via (at 84.582 64.008) (size 0.8) (drill 0.4) (layers F.Cu B.Cu) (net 1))
 (via (at 76.2 46.482) (size 0.4064) (drill 0.381) (layers F.Cu B.Cu) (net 1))
 (via (at 76.2 47.244) (size 0.4064) (drill 0.381) (layers F.Cu B.Cu) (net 1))
 (via (at 76.2 48.006) (size 0.4064) (drill 0.381) (layers F.Cu B.Cu) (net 1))
 (via (at 76.2 48.768) (size 0.4064) (drill 0.381) (layers F.Cu B.Cu) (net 1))
 (via (at 73.66 46.482) (size 0.4064) (drill 0.381) (layers F.Cu B.Cu) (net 1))
 (via (at 73.66 47.244) (size 0.4064) (drill 0.381) (layers F.Cu B.Cu) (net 1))
 (via (at 73.66 48.006) (size 0.4064) (drill 0.381) (layers F.Cu B.Cu) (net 1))
 (via (at 73.66 48.768) (size 0.4064) (drill 0.381) (layers F.Cu B.Cu) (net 1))
 (via (at 73.66 49.53) (size 0.4064) (drill 0.381) (layers F.Cu B.Cu) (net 1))
 (via (at 73.66 50.292) (size 0.4064) (drill 0.381) (layers F.Cu B.Cu) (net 1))
 (via (at 73.66 45.72) (size 0.4064) (drill 0.381) (layers F.Cu B.Cu) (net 1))
 (via (at 73.152 45.466) (size 0.4064) (drill 0.381) (layers F.Cu B.Cu) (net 1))
 (via (at 76.2 45.72) (size 0.4064) (drill 0.381) (layers F.Cu B.Cu) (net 1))
 (via (at 76.962 45.212) (size 0.4064) (drill 0.381) (layers F.Cu B.Cu) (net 1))
 (via (at 77.724 45.212) (size 0.4064) (drill 0.381) (layers F.Cu B.Cu) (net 1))
 (via (at 78.486 45.212) (size 0.4064) (drill 0.381) (layers F.Cu B.Cu) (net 1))
 (via (at 79.248 45.212) (size 0.4064) (drill 0.381) (layers F.Cu B.Cu) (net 1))
 (via (at 80.01 45.212) (size 0.4064) (drill 0.381) (layers F.Cu B.Cu) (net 1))
 (via (at 80.772 45.212) (size 0.4064) (drill 0.381) (layers F.Cu B.Cu) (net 1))
 (via (at 81.534 45.212) (size 0.4064) (drill 0.381) (layers F.Cu B.Cu) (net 1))
 (via (at 82.296 45.212) (size 0.4064) (drill 0.381) (layers F.Cu B.Cu) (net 1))
 (via (at 83.058 45.212) (size 0.4064) (drill 0.381) (layers F.Cu B.Cu) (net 1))
 (via (at 83.82 45.212) (size 0.4064) (drill 0.381) (layers F.Cu B.Cu) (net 1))
 (via (at 84.582 45.212) (size 0.4064) (drill 0.381) (layers F.Cu B.Cu) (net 1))
 (via (at 85.344 45.212) (size 0.4064) (drill 0.381) (layers F.Cu B.Cu) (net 1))
 (via (at 76.962 45.974) (size 0.4064) (drill 0.381) (layers F.Cu B.Cu) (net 1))
 (via (at 77.724 45.974) (size 0.4064) (drill 0.381) (layers F.Cu B.Cu) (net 1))
 (via (at 78.486 45.974) (size 0.4064) (drill 0.381) (layers F.Cu B.Cu) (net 1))
 (via (at 79.248 45.974) (size 0.4064) (drill 0.381) (layers F.Cu B.Cu) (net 1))
 (via (at 80.01 45.974) (size 0.4064) (drill 0.381) (layers F.Cu B.Cu) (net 1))
 (via (at 80.772 45.974) (size 0.4064) (drill 0.381) (layers F.Cu B.Cu) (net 1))
 (via (at 81.534 45.974) (size 0.4064) (drill 0.381) (layers F.Cu B.Cu) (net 1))
 (via (at 82.296 45.974) (size 0.4064) (drill 0.381) (layers F.Cu B.Cu) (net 1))
 (via (at 83.058 45.974) (size 0.4064) (drill 0.381) (layers F.Cu B.Cu) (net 1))
 (via (at 83.82 45.974) (size 0.4064) (drill 0.381) (layers F.Cu B.Cu) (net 1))
 (via (at 84.582 45.974) (size 0.4064) (drill 0.381) (layers F.Cu B.Cu) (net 1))
 (via (at 85.344 45.974) (size 0.4064) (drill 0.381) (layers F.Cu B.Cu) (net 1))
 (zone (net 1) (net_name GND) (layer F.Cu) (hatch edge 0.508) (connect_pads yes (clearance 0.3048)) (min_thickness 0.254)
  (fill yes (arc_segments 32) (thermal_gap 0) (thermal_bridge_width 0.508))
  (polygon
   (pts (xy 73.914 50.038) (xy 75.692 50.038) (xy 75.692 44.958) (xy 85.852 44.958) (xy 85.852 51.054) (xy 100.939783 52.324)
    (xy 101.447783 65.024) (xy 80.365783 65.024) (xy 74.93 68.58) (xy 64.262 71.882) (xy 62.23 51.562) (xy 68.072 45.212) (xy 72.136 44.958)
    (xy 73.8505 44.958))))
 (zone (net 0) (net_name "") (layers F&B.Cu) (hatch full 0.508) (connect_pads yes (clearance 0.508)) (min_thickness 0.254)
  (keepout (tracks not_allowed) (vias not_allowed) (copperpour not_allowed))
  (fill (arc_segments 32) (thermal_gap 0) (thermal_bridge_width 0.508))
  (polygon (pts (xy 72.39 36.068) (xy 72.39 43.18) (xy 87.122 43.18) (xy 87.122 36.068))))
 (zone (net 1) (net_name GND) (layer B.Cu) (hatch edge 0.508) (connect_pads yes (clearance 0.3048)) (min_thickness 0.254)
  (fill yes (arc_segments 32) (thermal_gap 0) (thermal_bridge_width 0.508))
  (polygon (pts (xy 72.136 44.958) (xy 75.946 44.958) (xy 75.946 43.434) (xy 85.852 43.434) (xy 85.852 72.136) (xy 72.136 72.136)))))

